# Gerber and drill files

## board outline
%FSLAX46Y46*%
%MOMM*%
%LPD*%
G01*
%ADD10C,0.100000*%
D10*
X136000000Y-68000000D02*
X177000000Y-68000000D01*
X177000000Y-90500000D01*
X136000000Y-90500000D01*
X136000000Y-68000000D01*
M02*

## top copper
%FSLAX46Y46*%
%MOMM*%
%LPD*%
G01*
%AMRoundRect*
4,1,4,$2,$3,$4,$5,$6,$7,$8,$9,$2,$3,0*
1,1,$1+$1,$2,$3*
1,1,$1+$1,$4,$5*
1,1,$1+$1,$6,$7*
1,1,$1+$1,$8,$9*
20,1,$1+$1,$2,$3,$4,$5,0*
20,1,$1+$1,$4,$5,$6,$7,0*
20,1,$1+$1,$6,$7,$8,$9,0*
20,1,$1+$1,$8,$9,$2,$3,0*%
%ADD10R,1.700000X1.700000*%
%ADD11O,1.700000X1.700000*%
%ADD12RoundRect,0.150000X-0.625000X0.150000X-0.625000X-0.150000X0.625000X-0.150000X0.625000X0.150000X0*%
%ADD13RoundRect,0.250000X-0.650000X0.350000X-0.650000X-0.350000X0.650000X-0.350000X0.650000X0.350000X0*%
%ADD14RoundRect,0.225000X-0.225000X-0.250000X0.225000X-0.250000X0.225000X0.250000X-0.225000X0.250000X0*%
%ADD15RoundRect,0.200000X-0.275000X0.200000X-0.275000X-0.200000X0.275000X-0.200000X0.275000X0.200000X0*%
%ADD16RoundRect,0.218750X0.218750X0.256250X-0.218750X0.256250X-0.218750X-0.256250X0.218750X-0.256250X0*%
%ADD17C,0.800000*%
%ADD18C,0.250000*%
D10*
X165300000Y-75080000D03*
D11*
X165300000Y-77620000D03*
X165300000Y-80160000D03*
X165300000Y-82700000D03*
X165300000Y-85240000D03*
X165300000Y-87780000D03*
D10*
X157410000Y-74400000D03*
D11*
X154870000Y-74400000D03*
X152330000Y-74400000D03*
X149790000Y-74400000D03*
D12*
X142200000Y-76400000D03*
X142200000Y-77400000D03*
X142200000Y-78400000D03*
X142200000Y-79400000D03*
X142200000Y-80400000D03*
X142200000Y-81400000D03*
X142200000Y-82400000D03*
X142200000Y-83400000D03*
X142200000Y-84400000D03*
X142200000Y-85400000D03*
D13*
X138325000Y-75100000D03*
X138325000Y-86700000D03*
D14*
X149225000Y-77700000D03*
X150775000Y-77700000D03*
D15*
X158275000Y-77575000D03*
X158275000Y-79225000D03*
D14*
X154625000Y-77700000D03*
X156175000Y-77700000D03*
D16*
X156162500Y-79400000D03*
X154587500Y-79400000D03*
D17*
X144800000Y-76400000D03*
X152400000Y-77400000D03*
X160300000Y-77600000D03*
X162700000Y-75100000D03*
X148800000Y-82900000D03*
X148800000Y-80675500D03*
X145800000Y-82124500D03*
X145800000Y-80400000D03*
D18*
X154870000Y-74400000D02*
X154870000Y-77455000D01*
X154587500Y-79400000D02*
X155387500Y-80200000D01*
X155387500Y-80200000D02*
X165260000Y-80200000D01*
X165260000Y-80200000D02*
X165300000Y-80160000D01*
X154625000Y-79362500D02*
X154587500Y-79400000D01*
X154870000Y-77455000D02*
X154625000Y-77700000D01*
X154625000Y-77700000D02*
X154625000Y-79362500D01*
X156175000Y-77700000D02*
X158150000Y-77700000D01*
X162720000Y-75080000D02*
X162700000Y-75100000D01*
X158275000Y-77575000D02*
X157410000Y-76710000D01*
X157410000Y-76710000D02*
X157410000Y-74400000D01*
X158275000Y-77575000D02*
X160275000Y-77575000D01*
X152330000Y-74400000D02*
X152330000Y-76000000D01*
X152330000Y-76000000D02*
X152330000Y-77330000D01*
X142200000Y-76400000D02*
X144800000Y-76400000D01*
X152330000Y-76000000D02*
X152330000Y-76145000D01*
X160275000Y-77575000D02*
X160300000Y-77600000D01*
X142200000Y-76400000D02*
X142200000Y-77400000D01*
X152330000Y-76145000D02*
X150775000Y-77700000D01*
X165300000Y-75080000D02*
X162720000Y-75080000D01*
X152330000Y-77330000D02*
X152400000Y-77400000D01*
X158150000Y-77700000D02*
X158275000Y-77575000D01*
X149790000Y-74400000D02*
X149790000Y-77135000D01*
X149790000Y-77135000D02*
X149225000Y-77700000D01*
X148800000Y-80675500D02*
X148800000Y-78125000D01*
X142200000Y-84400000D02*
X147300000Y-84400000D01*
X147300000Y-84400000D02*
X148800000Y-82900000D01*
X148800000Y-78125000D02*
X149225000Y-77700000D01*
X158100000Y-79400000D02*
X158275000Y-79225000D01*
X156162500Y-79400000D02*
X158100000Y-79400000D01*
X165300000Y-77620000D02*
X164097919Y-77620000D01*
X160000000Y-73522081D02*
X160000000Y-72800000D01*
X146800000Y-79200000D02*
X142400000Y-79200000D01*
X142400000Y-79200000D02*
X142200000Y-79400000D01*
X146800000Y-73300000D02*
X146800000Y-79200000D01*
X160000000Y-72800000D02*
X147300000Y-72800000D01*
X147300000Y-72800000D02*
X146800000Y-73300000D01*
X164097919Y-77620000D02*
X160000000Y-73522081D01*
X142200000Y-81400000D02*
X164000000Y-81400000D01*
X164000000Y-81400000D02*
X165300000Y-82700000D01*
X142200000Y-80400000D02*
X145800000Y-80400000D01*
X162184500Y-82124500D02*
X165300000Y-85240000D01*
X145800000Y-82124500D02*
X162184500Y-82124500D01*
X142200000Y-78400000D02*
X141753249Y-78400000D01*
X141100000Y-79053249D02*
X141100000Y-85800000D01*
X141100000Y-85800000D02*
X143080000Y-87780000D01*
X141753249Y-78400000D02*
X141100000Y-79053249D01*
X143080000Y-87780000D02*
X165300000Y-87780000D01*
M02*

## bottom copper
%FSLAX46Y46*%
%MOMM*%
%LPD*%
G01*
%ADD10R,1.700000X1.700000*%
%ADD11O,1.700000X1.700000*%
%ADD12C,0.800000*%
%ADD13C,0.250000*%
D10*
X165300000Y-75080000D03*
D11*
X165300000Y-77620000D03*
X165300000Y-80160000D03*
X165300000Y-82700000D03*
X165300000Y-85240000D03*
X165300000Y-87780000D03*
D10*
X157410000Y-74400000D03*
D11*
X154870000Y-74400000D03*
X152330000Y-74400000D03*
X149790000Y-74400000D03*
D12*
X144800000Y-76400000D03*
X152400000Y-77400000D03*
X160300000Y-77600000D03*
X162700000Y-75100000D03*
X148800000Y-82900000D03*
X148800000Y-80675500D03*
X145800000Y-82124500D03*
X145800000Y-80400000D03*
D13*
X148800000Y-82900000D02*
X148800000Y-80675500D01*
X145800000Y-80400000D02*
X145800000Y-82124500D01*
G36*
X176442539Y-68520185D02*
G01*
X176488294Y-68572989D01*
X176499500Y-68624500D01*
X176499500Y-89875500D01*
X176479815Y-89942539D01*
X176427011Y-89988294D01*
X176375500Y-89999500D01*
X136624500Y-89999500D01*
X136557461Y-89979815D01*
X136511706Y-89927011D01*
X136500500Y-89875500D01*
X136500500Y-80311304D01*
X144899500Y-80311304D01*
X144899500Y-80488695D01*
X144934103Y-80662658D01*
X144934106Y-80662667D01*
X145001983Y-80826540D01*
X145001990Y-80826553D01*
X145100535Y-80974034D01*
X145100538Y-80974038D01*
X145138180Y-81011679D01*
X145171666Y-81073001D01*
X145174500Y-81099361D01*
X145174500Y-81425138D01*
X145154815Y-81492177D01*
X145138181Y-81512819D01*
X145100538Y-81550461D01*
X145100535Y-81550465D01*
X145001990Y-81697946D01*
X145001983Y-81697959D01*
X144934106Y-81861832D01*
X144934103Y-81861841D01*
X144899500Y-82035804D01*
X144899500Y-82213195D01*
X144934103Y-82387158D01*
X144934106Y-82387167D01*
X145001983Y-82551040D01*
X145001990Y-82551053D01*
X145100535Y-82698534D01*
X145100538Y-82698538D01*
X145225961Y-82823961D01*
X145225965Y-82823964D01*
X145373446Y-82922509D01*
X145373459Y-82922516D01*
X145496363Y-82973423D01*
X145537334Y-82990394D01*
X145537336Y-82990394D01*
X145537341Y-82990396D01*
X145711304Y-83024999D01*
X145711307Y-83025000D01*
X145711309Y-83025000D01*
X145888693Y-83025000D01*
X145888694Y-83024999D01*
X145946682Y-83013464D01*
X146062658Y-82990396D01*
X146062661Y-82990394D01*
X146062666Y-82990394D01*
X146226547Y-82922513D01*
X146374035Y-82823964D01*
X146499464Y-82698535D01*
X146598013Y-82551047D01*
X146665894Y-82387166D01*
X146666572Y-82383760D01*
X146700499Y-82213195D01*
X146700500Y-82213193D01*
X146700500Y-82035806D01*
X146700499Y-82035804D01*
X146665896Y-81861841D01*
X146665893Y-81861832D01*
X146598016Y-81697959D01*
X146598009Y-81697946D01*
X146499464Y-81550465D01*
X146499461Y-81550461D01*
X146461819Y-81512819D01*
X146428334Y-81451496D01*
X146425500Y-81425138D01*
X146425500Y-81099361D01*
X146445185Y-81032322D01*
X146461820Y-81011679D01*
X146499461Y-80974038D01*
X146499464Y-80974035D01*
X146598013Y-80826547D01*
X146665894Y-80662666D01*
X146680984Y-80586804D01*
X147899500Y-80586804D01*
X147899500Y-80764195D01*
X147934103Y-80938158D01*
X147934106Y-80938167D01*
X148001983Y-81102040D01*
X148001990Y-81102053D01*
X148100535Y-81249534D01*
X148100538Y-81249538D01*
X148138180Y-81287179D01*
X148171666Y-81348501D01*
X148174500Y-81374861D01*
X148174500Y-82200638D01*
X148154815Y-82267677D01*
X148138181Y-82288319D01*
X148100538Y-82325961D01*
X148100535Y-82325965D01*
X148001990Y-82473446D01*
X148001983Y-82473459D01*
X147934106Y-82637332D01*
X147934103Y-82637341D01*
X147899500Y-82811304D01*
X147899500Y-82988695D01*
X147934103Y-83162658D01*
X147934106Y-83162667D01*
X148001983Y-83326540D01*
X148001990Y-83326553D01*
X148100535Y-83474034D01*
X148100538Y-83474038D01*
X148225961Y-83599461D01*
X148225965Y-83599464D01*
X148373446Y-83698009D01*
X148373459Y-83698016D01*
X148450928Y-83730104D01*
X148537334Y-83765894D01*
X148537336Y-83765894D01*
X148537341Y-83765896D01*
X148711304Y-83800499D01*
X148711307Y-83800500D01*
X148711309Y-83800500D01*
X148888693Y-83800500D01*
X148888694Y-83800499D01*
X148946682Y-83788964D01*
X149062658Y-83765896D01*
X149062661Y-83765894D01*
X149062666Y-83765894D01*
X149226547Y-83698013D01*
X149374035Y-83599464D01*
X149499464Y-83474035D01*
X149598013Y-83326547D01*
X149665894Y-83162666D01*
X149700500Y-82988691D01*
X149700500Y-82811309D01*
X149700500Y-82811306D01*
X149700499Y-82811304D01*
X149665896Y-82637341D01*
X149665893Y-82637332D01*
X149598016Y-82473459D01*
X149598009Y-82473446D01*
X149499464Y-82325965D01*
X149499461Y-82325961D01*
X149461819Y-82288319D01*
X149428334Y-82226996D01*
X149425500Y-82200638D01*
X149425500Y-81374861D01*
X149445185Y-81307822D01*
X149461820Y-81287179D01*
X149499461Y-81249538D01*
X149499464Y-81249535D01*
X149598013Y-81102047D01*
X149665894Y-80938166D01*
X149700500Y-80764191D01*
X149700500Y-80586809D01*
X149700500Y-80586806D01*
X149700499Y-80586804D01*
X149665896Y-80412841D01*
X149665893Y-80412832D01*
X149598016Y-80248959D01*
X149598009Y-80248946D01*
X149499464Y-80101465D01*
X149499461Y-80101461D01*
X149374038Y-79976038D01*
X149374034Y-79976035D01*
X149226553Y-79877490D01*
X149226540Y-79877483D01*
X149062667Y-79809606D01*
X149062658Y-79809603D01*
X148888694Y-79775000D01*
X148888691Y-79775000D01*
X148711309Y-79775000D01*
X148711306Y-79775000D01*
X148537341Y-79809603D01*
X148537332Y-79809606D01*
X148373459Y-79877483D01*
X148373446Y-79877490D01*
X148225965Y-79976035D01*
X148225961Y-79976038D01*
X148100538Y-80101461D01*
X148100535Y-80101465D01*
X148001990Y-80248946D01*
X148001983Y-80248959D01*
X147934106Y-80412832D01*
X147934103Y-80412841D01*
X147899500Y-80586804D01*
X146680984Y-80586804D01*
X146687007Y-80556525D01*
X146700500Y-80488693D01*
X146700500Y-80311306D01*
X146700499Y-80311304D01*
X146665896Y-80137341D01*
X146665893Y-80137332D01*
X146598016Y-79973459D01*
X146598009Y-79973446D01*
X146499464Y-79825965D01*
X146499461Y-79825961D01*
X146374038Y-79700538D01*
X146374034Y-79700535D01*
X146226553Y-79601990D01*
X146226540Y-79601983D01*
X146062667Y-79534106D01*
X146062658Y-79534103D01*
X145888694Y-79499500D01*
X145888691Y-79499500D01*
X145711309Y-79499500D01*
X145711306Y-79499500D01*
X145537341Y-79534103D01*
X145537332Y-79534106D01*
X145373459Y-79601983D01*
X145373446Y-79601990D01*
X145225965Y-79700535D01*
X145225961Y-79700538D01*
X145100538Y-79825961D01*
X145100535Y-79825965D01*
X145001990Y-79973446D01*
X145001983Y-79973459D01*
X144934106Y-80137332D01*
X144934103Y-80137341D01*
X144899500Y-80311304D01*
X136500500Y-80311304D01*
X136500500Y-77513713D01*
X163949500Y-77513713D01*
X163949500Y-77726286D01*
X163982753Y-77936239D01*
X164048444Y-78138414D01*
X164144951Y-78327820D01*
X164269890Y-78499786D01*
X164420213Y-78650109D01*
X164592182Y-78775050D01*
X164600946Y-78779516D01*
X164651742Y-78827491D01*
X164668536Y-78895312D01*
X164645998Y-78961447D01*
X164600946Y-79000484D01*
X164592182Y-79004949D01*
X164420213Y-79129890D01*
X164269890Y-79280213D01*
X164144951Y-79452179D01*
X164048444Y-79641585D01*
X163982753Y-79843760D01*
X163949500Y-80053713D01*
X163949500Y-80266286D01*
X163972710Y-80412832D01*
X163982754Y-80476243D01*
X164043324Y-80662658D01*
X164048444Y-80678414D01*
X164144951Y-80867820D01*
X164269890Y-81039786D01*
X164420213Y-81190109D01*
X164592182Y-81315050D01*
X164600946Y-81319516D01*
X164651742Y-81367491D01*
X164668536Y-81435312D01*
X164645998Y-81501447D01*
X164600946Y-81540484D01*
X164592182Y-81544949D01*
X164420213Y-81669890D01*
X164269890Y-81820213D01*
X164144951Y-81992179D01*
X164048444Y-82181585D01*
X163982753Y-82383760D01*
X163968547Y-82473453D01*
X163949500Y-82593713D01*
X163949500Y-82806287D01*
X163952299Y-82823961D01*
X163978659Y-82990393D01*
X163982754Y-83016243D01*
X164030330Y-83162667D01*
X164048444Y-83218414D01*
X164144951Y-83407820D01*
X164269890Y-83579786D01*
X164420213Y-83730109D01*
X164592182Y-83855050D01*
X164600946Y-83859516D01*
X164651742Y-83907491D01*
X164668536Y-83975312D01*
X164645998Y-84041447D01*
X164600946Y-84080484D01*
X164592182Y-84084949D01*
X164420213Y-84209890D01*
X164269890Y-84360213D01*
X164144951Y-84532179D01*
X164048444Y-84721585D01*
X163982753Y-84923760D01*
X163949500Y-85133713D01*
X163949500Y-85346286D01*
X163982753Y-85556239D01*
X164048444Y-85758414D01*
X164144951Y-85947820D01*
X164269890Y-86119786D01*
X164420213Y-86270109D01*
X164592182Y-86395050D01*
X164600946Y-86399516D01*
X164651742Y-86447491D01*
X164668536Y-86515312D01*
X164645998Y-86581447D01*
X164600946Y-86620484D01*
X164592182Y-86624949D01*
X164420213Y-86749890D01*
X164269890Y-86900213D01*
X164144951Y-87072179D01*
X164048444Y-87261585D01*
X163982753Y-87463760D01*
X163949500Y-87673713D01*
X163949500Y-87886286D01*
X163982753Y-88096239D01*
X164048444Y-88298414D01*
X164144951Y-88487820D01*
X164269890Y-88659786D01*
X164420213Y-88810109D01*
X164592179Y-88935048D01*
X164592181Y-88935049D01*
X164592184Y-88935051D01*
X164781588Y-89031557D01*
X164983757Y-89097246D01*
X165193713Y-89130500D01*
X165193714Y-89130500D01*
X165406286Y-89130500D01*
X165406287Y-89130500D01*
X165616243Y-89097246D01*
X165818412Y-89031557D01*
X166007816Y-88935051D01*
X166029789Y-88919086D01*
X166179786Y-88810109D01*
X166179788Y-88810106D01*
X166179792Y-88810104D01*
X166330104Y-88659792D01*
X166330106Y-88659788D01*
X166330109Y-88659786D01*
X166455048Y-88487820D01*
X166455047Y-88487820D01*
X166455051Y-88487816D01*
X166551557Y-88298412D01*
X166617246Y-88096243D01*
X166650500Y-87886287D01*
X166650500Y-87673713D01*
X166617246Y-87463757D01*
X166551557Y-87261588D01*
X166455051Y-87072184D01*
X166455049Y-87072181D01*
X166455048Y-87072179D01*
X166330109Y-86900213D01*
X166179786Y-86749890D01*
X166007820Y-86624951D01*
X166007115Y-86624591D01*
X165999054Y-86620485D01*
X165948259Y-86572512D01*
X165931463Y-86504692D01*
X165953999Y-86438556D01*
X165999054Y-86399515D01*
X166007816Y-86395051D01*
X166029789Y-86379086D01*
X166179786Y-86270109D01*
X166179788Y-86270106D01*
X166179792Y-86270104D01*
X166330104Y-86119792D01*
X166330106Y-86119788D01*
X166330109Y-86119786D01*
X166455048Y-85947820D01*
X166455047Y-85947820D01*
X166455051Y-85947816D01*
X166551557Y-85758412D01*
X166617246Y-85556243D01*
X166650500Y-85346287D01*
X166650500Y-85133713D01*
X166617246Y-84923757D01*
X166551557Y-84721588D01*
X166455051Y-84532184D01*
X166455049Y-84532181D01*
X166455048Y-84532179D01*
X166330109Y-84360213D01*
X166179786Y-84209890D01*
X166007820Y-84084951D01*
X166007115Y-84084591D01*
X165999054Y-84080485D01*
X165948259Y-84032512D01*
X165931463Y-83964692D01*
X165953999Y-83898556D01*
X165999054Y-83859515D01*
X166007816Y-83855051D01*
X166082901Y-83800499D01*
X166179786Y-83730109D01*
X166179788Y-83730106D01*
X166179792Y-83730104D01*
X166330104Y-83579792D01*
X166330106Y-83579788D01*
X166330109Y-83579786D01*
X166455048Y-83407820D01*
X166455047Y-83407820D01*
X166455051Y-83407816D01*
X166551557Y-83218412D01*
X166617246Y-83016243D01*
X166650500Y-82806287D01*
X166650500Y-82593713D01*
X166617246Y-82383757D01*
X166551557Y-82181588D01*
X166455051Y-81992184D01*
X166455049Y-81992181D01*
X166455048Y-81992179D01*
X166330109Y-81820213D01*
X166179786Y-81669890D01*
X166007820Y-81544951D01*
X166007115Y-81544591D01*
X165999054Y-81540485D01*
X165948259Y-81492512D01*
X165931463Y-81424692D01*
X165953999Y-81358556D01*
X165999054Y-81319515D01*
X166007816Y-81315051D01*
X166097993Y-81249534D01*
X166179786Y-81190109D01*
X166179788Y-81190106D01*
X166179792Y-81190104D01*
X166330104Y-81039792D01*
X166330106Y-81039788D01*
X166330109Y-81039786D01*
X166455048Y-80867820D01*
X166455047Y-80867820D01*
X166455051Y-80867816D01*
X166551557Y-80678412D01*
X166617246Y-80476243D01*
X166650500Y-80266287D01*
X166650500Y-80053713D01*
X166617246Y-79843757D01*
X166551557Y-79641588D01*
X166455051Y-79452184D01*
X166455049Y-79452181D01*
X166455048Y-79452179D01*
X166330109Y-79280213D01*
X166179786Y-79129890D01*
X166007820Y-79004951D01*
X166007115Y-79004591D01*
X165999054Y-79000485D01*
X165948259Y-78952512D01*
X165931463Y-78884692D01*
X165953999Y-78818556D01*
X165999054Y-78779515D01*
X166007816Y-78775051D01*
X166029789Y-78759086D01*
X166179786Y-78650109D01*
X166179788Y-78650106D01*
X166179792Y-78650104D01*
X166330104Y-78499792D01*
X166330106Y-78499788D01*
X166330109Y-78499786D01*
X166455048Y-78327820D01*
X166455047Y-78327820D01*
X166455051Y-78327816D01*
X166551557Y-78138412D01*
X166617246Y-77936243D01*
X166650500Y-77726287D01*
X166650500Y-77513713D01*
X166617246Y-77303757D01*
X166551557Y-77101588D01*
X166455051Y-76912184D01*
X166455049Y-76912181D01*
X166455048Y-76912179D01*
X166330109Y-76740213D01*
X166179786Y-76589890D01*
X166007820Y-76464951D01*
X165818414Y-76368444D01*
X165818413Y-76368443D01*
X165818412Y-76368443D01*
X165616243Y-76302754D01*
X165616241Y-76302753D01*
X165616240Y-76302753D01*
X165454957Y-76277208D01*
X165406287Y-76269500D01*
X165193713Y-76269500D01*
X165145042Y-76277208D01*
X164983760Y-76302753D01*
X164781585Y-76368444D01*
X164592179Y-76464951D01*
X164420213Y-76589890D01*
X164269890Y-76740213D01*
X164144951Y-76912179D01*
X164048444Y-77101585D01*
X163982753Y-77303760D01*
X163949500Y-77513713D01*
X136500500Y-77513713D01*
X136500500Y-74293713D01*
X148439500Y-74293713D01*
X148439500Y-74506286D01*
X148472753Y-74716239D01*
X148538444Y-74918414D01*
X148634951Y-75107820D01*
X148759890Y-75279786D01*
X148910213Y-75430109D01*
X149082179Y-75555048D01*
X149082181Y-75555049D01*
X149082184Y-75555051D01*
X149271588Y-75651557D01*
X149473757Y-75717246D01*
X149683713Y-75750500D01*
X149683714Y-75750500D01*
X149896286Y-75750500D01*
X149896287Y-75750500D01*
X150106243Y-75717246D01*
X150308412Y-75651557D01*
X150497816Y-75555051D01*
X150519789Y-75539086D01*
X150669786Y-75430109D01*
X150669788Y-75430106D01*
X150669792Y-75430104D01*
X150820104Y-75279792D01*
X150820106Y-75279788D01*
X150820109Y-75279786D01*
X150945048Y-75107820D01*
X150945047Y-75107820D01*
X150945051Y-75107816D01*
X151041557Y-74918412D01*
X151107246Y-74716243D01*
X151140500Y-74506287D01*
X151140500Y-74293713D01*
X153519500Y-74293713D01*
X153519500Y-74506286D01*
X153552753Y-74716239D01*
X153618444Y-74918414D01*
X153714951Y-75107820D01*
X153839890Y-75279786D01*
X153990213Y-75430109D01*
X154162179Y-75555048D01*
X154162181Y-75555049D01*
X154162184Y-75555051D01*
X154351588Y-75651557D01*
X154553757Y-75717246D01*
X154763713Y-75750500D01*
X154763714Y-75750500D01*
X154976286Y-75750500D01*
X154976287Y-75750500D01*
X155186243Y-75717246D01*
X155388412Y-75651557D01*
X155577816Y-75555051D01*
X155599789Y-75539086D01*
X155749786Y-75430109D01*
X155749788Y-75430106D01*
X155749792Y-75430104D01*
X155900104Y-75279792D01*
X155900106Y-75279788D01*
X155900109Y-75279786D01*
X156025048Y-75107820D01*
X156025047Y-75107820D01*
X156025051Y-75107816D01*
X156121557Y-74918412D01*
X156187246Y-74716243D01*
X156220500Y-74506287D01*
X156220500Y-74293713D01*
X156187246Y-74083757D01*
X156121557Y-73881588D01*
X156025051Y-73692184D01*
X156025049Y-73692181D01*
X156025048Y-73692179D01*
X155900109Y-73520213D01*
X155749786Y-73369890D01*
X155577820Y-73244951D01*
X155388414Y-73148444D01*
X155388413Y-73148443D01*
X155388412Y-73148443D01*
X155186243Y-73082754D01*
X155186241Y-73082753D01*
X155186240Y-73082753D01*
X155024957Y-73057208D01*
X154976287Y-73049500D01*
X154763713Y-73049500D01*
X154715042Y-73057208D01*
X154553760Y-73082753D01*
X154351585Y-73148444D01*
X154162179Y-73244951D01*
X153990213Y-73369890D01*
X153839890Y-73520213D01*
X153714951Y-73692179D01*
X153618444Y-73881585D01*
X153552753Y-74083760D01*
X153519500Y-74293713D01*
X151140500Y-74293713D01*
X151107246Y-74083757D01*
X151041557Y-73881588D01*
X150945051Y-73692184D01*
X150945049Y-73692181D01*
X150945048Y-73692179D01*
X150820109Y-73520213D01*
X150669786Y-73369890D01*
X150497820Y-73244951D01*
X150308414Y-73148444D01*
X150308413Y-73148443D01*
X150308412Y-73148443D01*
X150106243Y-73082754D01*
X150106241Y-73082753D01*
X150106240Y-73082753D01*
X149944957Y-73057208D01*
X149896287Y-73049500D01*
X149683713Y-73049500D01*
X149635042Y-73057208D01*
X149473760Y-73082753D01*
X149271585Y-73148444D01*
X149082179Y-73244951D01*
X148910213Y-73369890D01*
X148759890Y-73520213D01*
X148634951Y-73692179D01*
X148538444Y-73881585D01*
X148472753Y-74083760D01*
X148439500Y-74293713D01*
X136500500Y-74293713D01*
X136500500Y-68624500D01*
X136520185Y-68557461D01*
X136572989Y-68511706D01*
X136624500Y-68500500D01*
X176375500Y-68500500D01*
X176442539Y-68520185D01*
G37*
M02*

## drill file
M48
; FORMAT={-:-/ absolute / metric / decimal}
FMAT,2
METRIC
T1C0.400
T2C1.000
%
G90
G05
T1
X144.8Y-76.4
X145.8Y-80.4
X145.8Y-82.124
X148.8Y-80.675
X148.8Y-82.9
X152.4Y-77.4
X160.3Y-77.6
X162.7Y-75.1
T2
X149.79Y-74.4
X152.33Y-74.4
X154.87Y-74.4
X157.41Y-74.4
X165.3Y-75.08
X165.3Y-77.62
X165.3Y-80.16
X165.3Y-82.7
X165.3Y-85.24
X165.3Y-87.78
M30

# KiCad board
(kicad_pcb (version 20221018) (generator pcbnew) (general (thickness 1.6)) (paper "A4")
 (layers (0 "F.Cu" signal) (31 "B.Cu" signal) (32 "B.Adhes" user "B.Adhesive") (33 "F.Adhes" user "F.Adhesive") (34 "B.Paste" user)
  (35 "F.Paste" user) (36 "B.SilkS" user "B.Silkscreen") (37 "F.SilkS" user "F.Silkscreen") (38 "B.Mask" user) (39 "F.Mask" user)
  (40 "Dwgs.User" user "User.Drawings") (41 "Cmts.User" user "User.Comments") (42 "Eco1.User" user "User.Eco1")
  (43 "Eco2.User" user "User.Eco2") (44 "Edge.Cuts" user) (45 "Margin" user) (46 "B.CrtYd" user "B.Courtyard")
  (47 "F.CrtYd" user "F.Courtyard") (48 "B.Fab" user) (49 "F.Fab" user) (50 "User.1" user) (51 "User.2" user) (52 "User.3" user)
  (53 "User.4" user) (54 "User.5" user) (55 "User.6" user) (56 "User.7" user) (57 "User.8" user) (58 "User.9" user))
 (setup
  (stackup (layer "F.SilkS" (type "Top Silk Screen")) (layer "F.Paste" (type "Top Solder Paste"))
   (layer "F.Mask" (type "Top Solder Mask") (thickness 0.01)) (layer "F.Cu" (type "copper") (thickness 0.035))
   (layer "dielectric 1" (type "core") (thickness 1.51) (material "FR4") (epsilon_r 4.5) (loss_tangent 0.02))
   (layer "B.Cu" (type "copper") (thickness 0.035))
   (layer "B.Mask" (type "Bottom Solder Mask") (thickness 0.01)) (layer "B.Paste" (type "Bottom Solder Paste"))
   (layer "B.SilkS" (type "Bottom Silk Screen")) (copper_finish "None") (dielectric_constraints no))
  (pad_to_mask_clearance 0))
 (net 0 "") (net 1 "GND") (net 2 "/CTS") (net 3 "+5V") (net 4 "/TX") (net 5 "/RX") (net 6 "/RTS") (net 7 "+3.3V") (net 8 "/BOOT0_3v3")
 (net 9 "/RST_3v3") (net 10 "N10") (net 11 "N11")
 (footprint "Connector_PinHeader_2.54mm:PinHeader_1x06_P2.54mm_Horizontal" (layer "F.Cu") (at 165.3 75.08)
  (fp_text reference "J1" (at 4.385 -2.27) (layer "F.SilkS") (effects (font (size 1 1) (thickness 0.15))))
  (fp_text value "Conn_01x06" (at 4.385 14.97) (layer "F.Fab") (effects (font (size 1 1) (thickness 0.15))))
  (pad "1" thru_hole rect (at 0 0) (size 1.7 1.7) (drill 1) (layers "*.Cu" "*.Mask") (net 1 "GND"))
  (pad "2" thru_hole oval (at 0 2.54) (size 1.7 1.7) (drill 1) (layers "*.Cu" "*.Mask") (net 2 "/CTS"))
  (pad "3" thru_hole oval (at 0 5.08) (size 1.7 1.7) (drill 1) (layers "*.Cu" "*.Mask") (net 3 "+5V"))
  (pad "4" thru_hole oval (at 0 7.62) (size 1.7 1.7) (drill 1) (layers "*.Cu" "*.Mask") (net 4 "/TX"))
  (pad "5" thru_hole oval (at 0 10.16) (size 1.7 1.7) (drill 1) (layers "*.Cu" "*.Mask") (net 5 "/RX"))
  (pad "6" thru_hole oval (at 0 12.7) (size 1.7 1.7) (drill 1) (layers "*.Cu" "*.Mask") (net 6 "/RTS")))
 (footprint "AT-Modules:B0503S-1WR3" (layer "F.Cu") (at 153.6 72.3 180)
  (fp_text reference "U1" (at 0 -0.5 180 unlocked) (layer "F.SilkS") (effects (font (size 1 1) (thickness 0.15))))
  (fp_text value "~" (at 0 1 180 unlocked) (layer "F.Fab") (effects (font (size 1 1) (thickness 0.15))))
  (pad "1" thru_hole rect (at -3.81 -2.1 180) (size 1.7 1.7) (drill 1) (layers "*.Cu" "*.Mask") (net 1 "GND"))
  (pad "2" thru_hole oval (at -1.27 -2.1 180) (size 1.7 1.7) (drill 1) (layers "*.Cu" "*.Mask") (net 3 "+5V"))
  (pad "3" thru_hole oval (at 1.27 -2.1 180) (size 1.7 1.7) (drill 1) (layers "*.Cu" "*.Mask") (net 1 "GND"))
  (pad "4" thru_hole oval (at 3.81 -2.1 180) (size 1.7 1.7) (drill 1) (layers "*.Cu" "*.Mask") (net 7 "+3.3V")))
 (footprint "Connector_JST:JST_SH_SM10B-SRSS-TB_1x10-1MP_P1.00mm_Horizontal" (layer "F.Cu") (at 140.2 80.9 -90)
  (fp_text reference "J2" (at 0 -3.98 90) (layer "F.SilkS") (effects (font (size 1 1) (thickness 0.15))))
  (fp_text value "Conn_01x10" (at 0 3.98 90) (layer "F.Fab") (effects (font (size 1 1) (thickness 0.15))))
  (pad "1" smd roundrect (at -4.5 -2 270) (size 0.6 1.55) (layers "F.Cu" "F.Paste" "F.Mask") (roundrect_rratio 0.25) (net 1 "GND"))
  (pad "2" smd roundrect (at -3.5 -2 270) (size 0.6 1.55) (layers "F.Cu" "F.Paste" "F.Mask") (roundrect_rratio 0.25) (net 1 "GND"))
  (pad "3" smd roundrect (at -2.5 -2 270) (size 0.6 1.55) (layers "F.Cu" "F.Paste" "F.Mask") (roundrect_rratio 0.25) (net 6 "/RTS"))
  (pad "4" smd roundrect (at -1.5 -2 270) (size 0.6 1.55) (layers "F.Cu" "F.Paste" "F.Mask") (roundrect_rratio 0.25) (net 2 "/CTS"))
  (pad "5" smd roundrect (at -0.5 -2 270) (size 0.6 1.55) (layers "F.Cu" "F.Paste" "F.Mask") (roundrect_rratio 0.25) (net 5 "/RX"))
  (pad "6" smd roundrect (at 0.5 -2 270) (size 0.6 1.55) (layers "F.Cu" "F.Paste" "F.Mask") (roundrect_rratio 0.25) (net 4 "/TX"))
  (pad "7" smd roundrect (at 1.5 -2 270) (size 0.6 1.55) (layers "F.Cu" "F.Paste" "F.Mask") (roundrect_rratio 0.25) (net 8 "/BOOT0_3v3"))
  (pad "8" smd roundrect (at 2.5 -2 270) (size 0.6 1.55) (layers "F.Cu" "F.Paste" "F.Mask") (roundrect_rratio 0.25) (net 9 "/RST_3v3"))
  (pad "9" smd roundrect (at 3.5 -2 270) (size 0.6 1.55) (layers "F.Cu" "F.Paste" "F.Mask") (roundrect_rratio 0.25) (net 7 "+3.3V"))
  (pad "10" smd roundrect (at 4.5 -2 270) (size 0.6 1.55) (layers "F.Cu" "F.Paste" "F.Mask") (roundrect_rratio 0.25) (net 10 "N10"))
  (pad "MP" smd roundrect (at -5.8 1.875 270) (size 1.2 1.8) (layers "F.Cu" "F.Paste" "F.Mask") (roundrect_rratio 0.2083333333))
  (pad "MP" smd roundrect (at 5.8 1.875 270) (size 1.2 1.8) (layers "F.Cu" "F.Paste" "F.Mask") (roundrect_rratio 0.2083333333)))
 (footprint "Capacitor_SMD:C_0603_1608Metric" (layer "F.Cu") (at 150 77.7)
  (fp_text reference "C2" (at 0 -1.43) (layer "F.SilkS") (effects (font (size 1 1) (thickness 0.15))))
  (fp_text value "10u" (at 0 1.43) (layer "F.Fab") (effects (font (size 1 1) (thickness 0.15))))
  (pad "1" smd roundrect (at -0.775 0) (size 0.9 0.95) (layers "F.Cu" "F.Paste" "F.Mask") (roundrect_rratio 0.25) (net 7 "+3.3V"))
  (pad "2" smd roundrect (at 0.775 0) (size 0.9 0.95) (layers "F.Cu" "F.Paste" "F.Mask") (roundrect_rratio 0.25) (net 1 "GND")))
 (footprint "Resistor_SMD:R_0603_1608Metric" (layer "F.Cu") (at 158.275 78.4 -90)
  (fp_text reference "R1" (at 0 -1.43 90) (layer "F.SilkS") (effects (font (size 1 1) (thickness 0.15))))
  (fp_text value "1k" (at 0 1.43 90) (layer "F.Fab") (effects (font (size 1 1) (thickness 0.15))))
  (pad "1" smd roundrect (at -0.825 0 270) (size 0.8 0.95) (layers "F.Cu" "F.Paste" "F.Mask") (roundrect_rratio 0.25) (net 1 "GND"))
  (pad "2" smd roundrect (at 0.825 0 270) (size 0.8 0.95) (layers "F.Cu" "F.Paste" "F.Mask") (roundrect_rratio 0.25) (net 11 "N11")))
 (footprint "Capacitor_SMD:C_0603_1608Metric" (layer "F.Cu") (at 155.4 77.7)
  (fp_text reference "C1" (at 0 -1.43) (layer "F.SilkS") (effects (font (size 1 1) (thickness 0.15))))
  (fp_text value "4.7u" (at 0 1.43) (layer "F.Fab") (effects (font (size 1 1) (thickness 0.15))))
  (pad "1" smd roundrect (at -0.775 0) (size 0.9 0.95) (layers "F.Cu" "F.Paste" "F.Mask") (roundrect_rratio 0.25) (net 3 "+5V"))
  (pad "2" smd roundrect (at 0.775 0) (size 0.9 0.95) (layers "F.Cu" "F.Paste" "F.Mask") (roundrect_rratio 0.25) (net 1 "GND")))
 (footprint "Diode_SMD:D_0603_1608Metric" (layer "F.Cu") (at 155.375 79.4 180)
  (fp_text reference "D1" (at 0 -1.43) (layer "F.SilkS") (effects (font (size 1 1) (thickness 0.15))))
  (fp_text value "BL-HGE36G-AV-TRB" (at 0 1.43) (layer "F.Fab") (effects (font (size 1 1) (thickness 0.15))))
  (pad "1" smd roundrect (at -0.7875 0 180) (size 0.875 0.95) (layers "F.Cu" "F.Paste" "F.Mask") (roundrect_rratio 0.25) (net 11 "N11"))
  (pad "2" smd roundrect (at 0.7875 0 180) (size 0.875 0.95) (layers "F.Cu" "F.Paste" "F.Mask") (roundrect_rratio 0.25) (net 3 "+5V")))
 (gr_rect (start 136 68) (end 177 90.5) (stroke (width 0.1) (type default)) (fill none) (layer "Edge.Cuts"))
 (segment (start 154.87 74.4) (end 154.87 77.455) (width 0.25) (layer "F.Cu") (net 3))
 (segment (start 154.5875 79.4) (end 155.3875 80.2) (width 0.25) (layer "F.Cu") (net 3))
 (segment (start 155.3875 80.2) (end 165.26 80.2) (width 0.25) (layer "F.Cu") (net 3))
 (segment (start 165.26 80.2) (end 165.3 80.16) (width 0.25) (layer "F.Cu") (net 3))
 (segment (start 154.625 79.3625) (end 154.5875 79.4) (width 0.25) (layer "F.Cu") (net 3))
 (segment (start 154.87 77.455) (end 154.625 77.7) (width 0.25) (layer "F.Cu") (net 3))
 (segment (start 154.625 77.7) (end 154.625 79.3625) (width 0.25) (layer "F.Cu") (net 3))
 (segment (start 156.175 77.7) (end 158.15 77.7) (width 0.25) (layer "F.Cu") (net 1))
 (segment (start 162.72 75.08) (end 162.7 75.1) (width 0.25) (layer "F.Cu") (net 1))
 (segment (start 158.275 77.575) (end 157.41 76.71) (width 0.25) (layer "F.Cu") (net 1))
 (segment (start 157.41 76.71) (end 157.41 74.4) (width 0.25) (layer "F.Cu") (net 1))
 (segment (start 158.275 77.575) (end 160.275 77.575) (width 0.25) (layer "F.Cu") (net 1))
 (segment (start 152.33 74.4) (end 152.33 76) (width 0.25) (layer "F.Cu") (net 1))
 (segment (start 152.33 76) (end 152.33 77.33) (width 0.25) (layer "F.Cu") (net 1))
 (segment (start 142.2 76.4) (end 144.8 76.4) (width 0.25) (layer "F.Cu") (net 1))
 (segment (start 152.33 76) (end 152.33 76.145) (width 0.25) (layer "F.Cu") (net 1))
 (segment (start 160.275 77.575) (end 160.3 77.6) (width 0.25) (layer "F.Cu") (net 1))
 (segment (start 142.2 76.4) (end 142.2 77.4) (width 0.25) (layer "F.Cu") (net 1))
 (segment (start 152.33 76.145) (end 150.775 77.7) (width 0.25) (layer "F.Cu") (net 1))
 (segment (start 165.3 75.08) (end 162.72 75.08) (width 0.25) (layer "F.Cu") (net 1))
 (segment (start 152.33 77.33) (end 152.4 77.4) (width 0.25) (layer "F.Cu") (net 1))
 (segment (start 158.15 77.7) (end 158.275 77.575) (width 0.25) (layer "F.Cu") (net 1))
 (via (at 144.8 76.4) (size 0.8) (drill 0.4) (layers "F.Cu" "B.Cu") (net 1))
 (via (at 152.4 77.4) (size 0.8) (drill 0.4) (layers "F.Cu" "B.Cu") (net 1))
 (via (at 160.3 77.6) (size 0.8) (drill 0.4) (layers "F.Cu" "B.Cu") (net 1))
 (via (at 162.7 75.1) (size 0.8) (drill 0.4) (layers "F.Cu" "B.Cu") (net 1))
 (segment (start 149.79 74.4) (end 149.79 77.135) (width 0.25) (layer "F.Cu") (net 7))
 (segment (start 149.79 77.135) (end 149.225 77.7) (width 0.25) (layer "F.Cu") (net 7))
 (segment (start 148.8 80.6755) (end 148.8 78.125) (width 0.25) (layer "F.Cu") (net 7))
 (segment (start 142.2 84.4) (end 147.3 84.4) (width 0.25) (layer "F.Cu") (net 7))
 (segment (start 147.3 84.4) (end 148.8 82.9) (width 0.25) (layer "F.Cu") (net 7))
 (segment (start 148.8 78.125) (end 149.225 77.7) (width 0.25) (layer "F.Cu") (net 7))
 (via (at 148.8 82.9) (size 0.8) (drill 0.4) (layers "F.Cu" "B.Cu") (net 7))
 (via (at 148.8 80.6755) (size 0.8) (drill 0.4) (layers "F.Cu" "B.Cu") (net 7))
 (segment (start 148.8 82.9) (end 148.8 80.6755) (width 0.25) (layer "B.Cu") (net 7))
 (segment (start 158.1 79.4) (end 158.275 79.225) (width 0.25) (layer "F.Cu") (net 11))
 (segment (start 156.1625 79.4) (end 158.1 79.4) (width 0.25) (layer "F.Cu") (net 11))
 (segment (start 165.3 77.62) (end 164.097919 77.62) (width 0.25) (layer "F.Cu") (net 2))
 (segment (start 160 73.522081) (end 160 72.8) (width 0.25) (layer "F.Cu") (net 2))
 (segment (start 146.8 79.2) (end 142.4 79.2) (width 0.25) (layer "F.Cu") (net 2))
 (segment (start 142.4 79.2) (end 142.2 79.4) (width 0.25) (layer "F.Cu") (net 2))
 (segment (start 146.8 73.3) (end 146.8 79.2) (width 0.25) (layer "F.Cu") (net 2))
 (segment (start 160 72.8) (end 147.3 72.8) (width 0.25) (layer "F.Cu") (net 2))
 (segment (start 147.3 72.8) (end 146.8 73.3) (width 0.25) (layer "F.Cu") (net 2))
 (segment (start 164.097919 77.62) (end 160 73.522081) (width 0.25) (layer "F.Cu") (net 2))
 (segment (start 142.2 81.4) (end 164 81.4) (width 0.25) (layer "F.Cu") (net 4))
 (segment (start 164 81.4) (end 165.3 82.7) (width 0.25) (layer "F.Cu") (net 4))
 (segment (start 142.2 80.4) (end 145.8 80.4) (width 0.25) (layer "F.Cu") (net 5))
 (segment (start 162.1845 82.1245) (end 165.3 85.24) (width 0.25) (layer "F.Cu") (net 5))
 (segment (start 145.8 82.1245) (end 162.1845 82.1245) (width 0.25) (layer "F.Cu") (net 5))
 (via (at 145.8 82.1245) (size 0.8) (drill 0.4) (layers "F.Cu" "B.Cu") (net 5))
 (via (at 145.8 80.4) (size 0.8) (drill 0.4) (layers "F.Cu" "B.Cu") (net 5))
 (segment (start 145.8 80.4) (end 145.8 82.1245) (width 0.25) (layer "B.Cu") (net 5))
 (segment (start 142.2 78.4) (end 141.753249 78.4) (width 0.25) (layer "F.Cu") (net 6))
 (segment (start 141.1 79.053249) (end 141.1 85.8) (width 0.25) (layer "F.Cu") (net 6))
 (segment (start 141.1 85.8) (end 143.08 87.78) (width 0.25) (layer "F.Cu") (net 6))
 (segment (start 141.753249 78.4) (end 141.1 79.053249) (width 0.25) (layer "F.Cu") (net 6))
 (segment (start 143.08 87.78) (end 165.3 87.78) (width 0.25) (layer "F.Cu") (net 6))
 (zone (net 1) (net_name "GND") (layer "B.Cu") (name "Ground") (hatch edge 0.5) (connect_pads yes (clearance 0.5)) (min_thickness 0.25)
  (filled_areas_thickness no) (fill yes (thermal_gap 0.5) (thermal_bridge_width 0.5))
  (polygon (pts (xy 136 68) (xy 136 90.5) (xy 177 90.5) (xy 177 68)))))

